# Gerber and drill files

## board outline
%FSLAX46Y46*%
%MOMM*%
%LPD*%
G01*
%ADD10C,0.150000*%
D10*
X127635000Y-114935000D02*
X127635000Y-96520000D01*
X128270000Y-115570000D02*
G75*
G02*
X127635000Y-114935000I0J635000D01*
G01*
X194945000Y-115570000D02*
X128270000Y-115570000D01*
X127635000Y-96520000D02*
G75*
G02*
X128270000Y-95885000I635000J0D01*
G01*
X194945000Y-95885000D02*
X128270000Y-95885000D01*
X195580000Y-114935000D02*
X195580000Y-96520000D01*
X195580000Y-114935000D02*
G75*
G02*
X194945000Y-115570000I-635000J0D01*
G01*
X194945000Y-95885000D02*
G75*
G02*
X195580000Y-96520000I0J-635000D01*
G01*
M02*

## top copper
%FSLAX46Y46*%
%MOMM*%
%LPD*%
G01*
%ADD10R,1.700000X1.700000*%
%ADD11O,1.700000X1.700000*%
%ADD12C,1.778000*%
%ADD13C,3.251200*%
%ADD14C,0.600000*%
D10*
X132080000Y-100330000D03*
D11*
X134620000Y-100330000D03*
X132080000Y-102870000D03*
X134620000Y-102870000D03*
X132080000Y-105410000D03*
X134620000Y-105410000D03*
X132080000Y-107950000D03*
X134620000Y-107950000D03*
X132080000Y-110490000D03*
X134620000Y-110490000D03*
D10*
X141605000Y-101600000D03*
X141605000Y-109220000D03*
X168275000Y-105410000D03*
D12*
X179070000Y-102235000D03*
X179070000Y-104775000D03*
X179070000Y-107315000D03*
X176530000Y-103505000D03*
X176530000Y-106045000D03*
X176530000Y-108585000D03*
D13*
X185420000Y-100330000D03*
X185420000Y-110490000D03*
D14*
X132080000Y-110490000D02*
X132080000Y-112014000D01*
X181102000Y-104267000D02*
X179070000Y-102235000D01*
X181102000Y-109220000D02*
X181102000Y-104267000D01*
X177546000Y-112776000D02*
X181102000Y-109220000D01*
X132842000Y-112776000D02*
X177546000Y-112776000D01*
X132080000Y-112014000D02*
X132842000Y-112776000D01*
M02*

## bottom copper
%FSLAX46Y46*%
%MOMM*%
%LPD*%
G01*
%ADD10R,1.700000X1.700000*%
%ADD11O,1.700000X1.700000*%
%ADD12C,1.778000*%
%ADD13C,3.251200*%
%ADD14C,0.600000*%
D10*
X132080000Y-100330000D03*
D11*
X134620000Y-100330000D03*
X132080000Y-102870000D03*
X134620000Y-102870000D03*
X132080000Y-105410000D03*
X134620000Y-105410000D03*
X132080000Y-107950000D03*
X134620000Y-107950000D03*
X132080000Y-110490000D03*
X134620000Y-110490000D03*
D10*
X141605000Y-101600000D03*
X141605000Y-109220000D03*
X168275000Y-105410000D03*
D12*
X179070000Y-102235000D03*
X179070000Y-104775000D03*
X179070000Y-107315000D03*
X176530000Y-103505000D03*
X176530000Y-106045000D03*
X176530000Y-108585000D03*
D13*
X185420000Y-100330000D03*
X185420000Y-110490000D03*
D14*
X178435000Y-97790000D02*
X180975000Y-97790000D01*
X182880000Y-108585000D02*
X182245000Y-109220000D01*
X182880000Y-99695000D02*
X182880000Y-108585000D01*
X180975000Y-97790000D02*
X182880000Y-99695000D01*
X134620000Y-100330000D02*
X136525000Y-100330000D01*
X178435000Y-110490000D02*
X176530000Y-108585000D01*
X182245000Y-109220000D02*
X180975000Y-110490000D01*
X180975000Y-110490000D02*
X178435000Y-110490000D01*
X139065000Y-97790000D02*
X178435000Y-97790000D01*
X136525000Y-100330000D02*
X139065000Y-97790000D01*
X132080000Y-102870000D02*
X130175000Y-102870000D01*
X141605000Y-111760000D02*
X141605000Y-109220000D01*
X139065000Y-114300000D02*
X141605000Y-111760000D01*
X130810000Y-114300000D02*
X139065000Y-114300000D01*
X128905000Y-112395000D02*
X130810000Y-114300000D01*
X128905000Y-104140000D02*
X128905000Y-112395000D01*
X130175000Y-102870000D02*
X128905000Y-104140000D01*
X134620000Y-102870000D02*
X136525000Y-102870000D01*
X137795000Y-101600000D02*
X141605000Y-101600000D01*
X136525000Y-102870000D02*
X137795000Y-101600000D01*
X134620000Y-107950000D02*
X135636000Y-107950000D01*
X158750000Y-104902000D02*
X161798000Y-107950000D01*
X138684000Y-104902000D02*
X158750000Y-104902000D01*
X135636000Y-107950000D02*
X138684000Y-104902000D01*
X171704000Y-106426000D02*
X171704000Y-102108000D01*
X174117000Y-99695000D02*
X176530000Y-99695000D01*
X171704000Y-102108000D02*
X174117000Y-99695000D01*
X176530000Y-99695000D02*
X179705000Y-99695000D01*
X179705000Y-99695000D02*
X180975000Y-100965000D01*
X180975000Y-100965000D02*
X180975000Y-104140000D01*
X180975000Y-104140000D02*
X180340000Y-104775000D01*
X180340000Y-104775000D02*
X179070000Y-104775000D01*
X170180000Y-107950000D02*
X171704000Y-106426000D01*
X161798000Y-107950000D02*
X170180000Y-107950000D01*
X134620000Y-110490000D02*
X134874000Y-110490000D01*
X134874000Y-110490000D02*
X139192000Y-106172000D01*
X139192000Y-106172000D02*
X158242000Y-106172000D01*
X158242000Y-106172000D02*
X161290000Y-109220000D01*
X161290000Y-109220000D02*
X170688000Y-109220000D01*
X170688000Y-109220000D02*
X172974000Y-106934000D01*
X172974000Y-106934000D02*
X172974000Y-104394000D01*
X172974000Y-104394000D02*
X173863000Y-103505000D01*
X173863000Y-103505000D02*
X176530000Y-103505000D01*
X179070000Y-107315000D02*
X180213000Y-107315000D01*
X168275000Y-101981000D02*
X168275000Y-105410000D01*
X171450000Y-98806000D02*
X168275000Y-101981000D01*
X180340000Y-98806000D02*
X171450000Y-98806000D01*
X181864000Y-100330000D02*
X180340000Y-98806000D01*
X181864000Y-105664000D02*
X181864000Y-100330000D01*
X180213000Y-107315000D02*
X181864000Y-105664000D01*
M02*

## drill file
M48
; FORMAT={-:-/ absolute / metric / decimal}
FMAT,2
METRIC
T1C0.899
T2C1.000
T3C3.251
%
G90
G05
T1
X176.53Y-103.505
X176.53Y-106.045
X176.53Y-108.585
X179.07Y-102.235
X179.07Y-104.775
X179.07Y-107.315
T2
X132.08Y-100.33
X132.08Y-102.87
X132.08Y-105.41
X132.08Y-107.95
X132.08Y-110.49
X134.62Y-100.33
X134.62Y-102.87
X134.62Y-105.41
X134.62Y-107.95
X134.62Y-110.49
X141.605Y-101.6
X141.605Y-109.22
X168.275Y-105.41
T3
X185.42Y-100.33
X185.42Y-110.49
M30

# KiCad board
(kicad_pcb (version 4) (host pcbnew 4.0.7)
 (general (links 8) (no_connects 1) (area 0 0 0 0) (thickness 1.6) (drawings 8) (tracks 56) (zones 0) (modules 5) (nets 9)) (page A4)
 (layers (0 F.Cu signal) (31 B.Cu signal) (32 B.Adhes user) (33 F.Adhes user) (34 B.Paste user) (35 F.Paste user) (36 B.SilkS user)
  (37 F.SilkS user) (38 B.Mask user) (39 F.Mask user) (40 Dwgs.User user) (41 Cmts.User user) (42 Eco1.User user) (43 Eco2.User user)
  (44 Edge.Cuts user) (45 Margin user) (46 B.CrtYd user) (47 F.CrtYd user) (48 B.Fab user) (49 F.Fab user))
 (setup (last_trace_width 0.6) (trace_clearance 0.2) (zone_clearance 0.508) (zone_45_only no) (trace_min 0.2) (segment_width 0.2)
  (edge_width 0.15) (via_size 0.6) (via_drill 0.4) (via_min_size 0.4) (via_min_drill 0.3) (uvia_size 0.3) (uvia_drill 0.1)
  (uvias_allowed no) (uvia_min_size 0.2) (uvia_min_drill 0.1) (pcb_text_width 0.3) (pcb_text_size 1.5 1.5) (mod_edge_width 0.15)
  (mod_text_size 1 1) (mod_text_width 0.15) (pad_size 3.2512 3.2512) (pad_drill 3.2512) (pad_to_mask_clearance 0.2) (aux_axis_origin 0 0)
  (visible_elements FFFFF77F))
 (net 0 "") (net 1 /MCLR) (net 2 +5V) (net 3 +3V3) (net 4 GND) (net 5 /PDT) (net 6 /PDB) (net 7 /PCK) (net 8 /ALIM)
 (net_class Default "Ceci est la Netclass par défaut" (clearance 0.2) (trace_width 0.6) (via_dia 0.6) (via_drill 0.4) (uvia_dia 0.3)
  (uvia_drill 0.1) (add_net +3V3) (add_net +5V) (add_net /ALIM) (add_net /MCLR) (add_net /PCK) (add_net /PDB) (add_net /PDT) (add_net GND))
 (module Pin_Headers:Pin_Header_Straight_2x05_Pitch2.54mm (layer F.Cu) (at 132.08 100.33)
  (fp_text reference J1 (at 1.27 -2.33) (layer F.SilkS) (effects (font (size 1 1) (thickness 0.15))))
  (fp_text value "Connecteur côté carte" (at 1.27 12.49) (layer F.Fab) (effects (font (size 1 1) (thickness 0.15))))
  (pad 1 thru_hole rect (at 0 0) (size 1.7 1.7) (drill 1) (layers *.Cu *.Mask))
  (pad 2 thru_hole oval (at 2.54 0) (size 1.7 1.7) (drill 1) (layers *.Cu *.Mask) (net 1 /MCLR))
  (pad 3 thru_hole oval (at 0 2.54) (size 1.7 1.7) (drill 1) (layers *.Cu *.Mask) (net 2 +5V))
  (pad 4 thru_hole oval (at 2.54 2.54) (size 1.7 1.7) (drill 1) (layers *.Cu *.Mask) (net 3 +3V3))
  (pad 5 thru_hole oval (at 0 5.08) (size 1.7 1.7) (drill 1) (layers *.Cu *.Mask))
  (pad 6 thru_hole oval (at 2.54 5.08) (size 1.7 1.7) (drill 1) (layers *.Cu *.Mask) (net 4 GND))
  (pad 7 thru_hole oval (at 0 7.62) (size 1.7 1.7) (drill 1) (layers *.Cu *.Mask))
  (pad 8 thru_hole oval (at 2.54 7.62) (size 1.7 1.7) (drill 1) (layers *.Cu *.Mask) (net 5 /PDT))
  (pad 9 thru_hole oval (at 0 10.16) (size 1.7 1.7) (drill 1) (layers *.Cu *.Mask) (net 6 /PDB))
  (pad 10 thru_hole oval (at 2.54 10.16) (size 1.7 1.7) (drill 1) (layers *.Cu *.Mask) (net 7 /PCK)))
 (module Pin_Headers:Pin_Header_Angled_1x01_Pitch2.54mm (layer F.Cu) (at 141.605 101.6)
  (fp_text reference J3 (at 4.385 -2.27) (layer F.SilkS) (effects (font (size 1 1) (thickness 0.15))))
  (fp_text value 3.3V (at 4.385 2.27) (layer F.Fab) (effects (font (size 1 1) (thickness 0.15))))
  (pad 1 thru_hole rect (at 0 0) (size 1.7 1.7) (drill 1) (layers *.Cu *.Mask) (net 3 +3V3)))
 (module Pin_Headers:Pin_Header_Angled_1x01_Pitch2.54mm (layer F.Cu) (at 141.605 109.22)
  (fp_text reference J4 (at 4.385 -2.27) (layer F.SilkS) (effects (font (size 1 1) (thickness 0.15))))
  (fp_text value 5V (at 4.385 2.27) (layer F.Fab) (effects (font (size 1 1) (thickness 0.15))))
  (pad 1 thru_hole rect (at 0 0) (size 1.7 1.7) (drill 1) (layers *.Cu *.Mask) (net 2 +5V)))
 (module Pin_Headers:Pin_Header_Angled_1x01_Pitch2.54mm (layer F.Cu) (at 168.275 105.41 180)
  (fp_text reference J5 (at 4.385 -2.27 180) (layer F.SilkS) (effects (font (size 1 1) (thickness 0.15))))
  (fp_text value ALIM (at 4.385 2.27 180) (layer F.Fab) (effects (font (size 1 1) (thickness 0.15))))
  (pad 1 thru_hole rect (at 0 0 180) (size 1.7 1.7) (drill 1) (layers *.Cu *.Mask) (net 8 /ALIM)))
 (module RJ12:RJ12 (layer F.Cu) (at 185.42 105.41 270)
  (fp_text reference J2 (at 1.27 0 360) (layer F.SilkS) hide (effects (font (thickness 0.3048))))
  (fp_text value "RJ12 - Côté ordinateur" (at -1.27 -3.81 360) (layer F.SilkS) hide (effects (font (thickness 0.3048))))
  (pad 6 thru_hole circle (at -3.175 6.35 270) (size 1.778 1.778) (drill 0.89916) (layers *.Cu *.Mask F.SilkS) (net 6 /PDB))
  (pad 4 thru_hole circle (at -0.635 6.35 270) (size 1.778 1.778) (drill 0.89916) (layers *.Cu *.Mask F.SilkS) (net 5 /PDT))
  (pad 2 thru_hole circle (at 1.905 6.35 270) (size 1.778 1.778) (drill 0.89916) (layers *.Cu *.Mask F.SilkS) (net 8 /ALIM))
  (pad 5 thru_hole circle (at -1.905 8.89 270) (size 1.778 1.778) (drill 0.89916) (layers *.Cu *.Mask F.SilkS) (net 7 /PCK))
  (pad 3 thru_hole circle (at 0.635 8.89 270) (size 1.778 1.778) (drill 0.89916) (layers *.Cu *.Mask F.SilkS) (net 4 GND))
  (pad 1 thru_hole circle (at 3.175 8.89 270) (size 1.778 1.778) (drill 0.89916) (layers *.Cu *.Mask F.SilkS) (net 1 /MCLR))
  (pad 8 thru_hole circle (at -5.08 0 270) (size 3.2512 3.2512) (drill 3.2512) (layers *.Cu *.Mask F.SilkS))
  (pad 7 thru_hole circle (at 5.08 0 270) (size 3.2512 3.2512) (drill 3.2512) (layers *.Cu *.Mask F.SilkS)))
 (gr_line (start 127.635 114.935) (end 127.635 96.52) (angle 90) (layer Edge.Cuts) (width 0.15))
 (gr_arc (start 128.27 114.935) (end 128.27 115.57) (angle 90) (layer Edge.Cuts) (width 0.15))
 (gr_line (start 194.945 115.57) (end 128.27 115.57) (angle 90) (layer Edge.Cuts) (width 0.15))
 (gr_arc (start 128.27 96.52) (end 127.635 96.52) (angle 90) (layer Edge.Cuts) (width 0.15))
 (gr_line (start 194.945 95.885) (end 128.27 95.885) (angle 90) (layer Edge.Cuts) (width 0.15))
 (gr_line (start 195.58 114.935) (end 195.58 96.52) (angle 90) (layer Edge.Cuts) (width 0.15))
 (gr_arc (start 194.945 114.935) (end 195.58 114.935) (angle 90) (layer Edge.Cuts) (width 0.15))
 (gr_arc (start 194.945 96.52) (end 194.945 95.885) (angle 90) (layer Edge.Cuts) (width 0.15))
 (segment (start 178.435 97.79) (end 180.975 97.79) (width 0.6) (layer B.Cu) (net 1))
 (segment (start 182.88 108.585) (end 182.245 109.22) (width 0.6) (layer B.Cu) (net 1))
 (segment (start 182.88 99.695) (end 182.88 108.585) (width 0.6) (layer B.Cu) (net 1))
 (segment (start 180.975 97.79) (end 182.88 99.695) (width 0.6) (layer B.Cu) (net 1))
 (segment (start 134.62 100.33) (end 136.525 100.33) (width 0.6) (layer B.Cu) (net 1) (status 400000))
 (segment (start 178.435 110.49) (end 176.53 108.585) (width 0.6) (layer B.Cu) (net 1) (status 800000))
 (segment (start 182.245 109.22) (end 180.975 110.49) (width 0.6) (layer B.Cu) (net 1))
 (segment (start 180.975 110.49) (end 178.435 110.49) (width 0.6) (layer B.Cu) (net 1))
 (segment (start 139.065 97.79) (end 178.435 97.79) (width 0.6) (layer B.Cu) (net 1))
 (segment (start 136.525 100.33) (end 139.065 97.79) (width 0.6) (layer B.Cu) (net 1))
 (segment (start 132.08 102.87) (end 130.175 102.87) (width 0.6) (layer B.Cu) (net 2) (status 400000))
 (segment (start 141.605 111.76) (end 141.605 109.22) (width 0.6) (layer B.Cu) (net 2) (status 800000))
 (segment (start 139.065 114.3) (end 141.605 111.76) (width 0.6) (layer B.Cu) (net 2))
 (segment (start 130.81 114.3) (end 139.065 114.3) (width 0.6) (layer B.Cu) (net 2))
 (segment (start 128.905 112.395) (end 130.81 114.3) (width 0.6) (layer B.Cu) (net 2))
 (segment (start 128.905 104.14) (end 128.905 112.395) (width 0.6) (layer B.Cu) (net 2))
 (segment (start 130.175 102.87) (end 128.905 104.14) (width 0.6) (layer B.Cu) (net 2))
 (segment (start 134.62 102.87) (end 136.525 102.87) (width 0.6) (layer B.Cu) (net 3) (status 400000))
 (segment (start 137.795 101.6) (end 141.605 101.6) (width 0.6) (layer B.Cu) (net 3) (status 800000))
 (segment (start 136.525 102.87) (end 137.795 101.6) (width 0.6) (layer B.Cu) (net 3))
 (segment (start 134.62 107.95) (end 135.636 107.95) (width 0.6) (layer B.Cu) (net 5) (status 400000))
 (segment (start 158.75 104.902) (end 161.798 107.95) (width 0.6) (layer B.Cu) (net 5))
 (segment (start 138.684 104.902) (end 158.75 104.902) (width 0.6) (layer B.Cu) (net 5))
 (segment (start 135.636 107.95) (end 138.684 104.902) (width 0.6) (layer B.Cu) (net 5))
 (segment (start 171.704 106.426) (end 171.704 102.108) (width 0.6) (layer B.Cu) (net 5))
 (segment (start 174.117 99.695) (end 176.53 99.695) (width 0.6) (layer B.Cu) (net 5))
 (segment (start 171.704 102.108) (end 174.117 99.695) (width 0.6) (layer B.Cu) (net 5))
 (segment (start 176.53 99.695) (end 179.705 99.695) (width 0.6) (layer B.Cu) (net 5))
 (segment (start 179.705 99.695) (end 180.975 100.965) (width 0.6) (layer B.Cu) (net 5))
 (segment (start 180.975 100.965) (end 180.975 104.14) (width 0.6) (layer B.Cu) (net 5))
 (segment (start 180.975 104.14) (end 180.34 104.775) (width 0.6) (layer B.Cu) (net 5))
 (segment (start 180.34 104.775) (end 179.07 104.775) (width 0.6) (layer B.Cu) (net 5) (status 800000))
 (segment (start 170.18 107.95) (end 171.704 106.426) (width 0.6) (layer B.Cu) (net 5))
 (segment (start 161.798 107.95) (end 170.18 107.95) (width 0.6) (layer B.Cu) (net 5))
 (segment (start 132.08 110.49) (end 132.08 112.014) (width 0.6) (layer F.Cu) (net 6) (status 400000))
 (segment (start 181.102 104.267) (end 179.07 102.235) (width 0.6) (layer F.Cu) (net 6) (status 800000))
 (segment (start 181.102 109.22) (end 181.102 104.267) (width 0.6) (layer F.Cu) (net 6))
 (segment (start 177.546 112.776) (end 181.102 109.22) (width 0.6) (layer F.Cu) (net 6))
 (segment (start 132.842 112.776) (end 177.546 112.776) (width 0.6) (layer F.Cu) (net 6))
 (segment (start 132.08 112.014) (end 132.842 112.776) (width 0.6) (layer F.Cu) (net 6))
 (segment (start 134.62 110.49) (end 134.874 110.49) (width 0.6) (layer B.Cu) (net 7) (status C00000))
 (segment (start 134.874 110.49) (end 139.192 106.172) (width 0.6) (layer B.Cu) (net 7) (status 400000))
 (segment (start 139.192 106.172) (end 158.242 106.172) (width 0.6) (layer B.Cu) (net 7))
 (segment (start 158.242 106.172) (end 161.29 109.22) (width 0.6) (layer B.Cu) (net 7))
 (segment (start 161.29 109.22) (end 170.688 109.22) (width 0.6) (layer B.Cu) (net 7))
 (segment (start 170.688 109.22) (end 172.974 106.934) (width 0.6) (layer B.Cu) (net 7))
 (segment (start 172.974 106.934) (end 172.974 104.394) (width 0.6) (layer B.Cu) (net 7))
 (segment (start 172.974 104.394) (end 173.863 103.505) (width 0.6) (layer B.Cu) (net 7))
 (segment (start 173.863 103.505) (end 176.53 103.505) (width 0.6) (layer B.Cu) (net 7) (status 800000))
 (segment (start 179.07 107.315) (end 180.213 107.315) (width 0.6) (layer B.Cu) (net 8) (status 400000))
 (segment (start 168.275 101.981) (end 168.275 105.41) (width 0.6) (layer B.Cu) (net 8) (status 800000))
 (segment (start 171.45 98.806) (end 168.275 101.981) (width 0.6) (layer B.Cu) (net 8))
 (segment (start 180.34 98.806) (end 171.45 98.806) (width 0.6) (layer B.Cu) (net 8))
 (segment (start 181.864 100.33) (end 180.34 98.806) (width 0.6) (layer B.Cu) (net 8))
 (segment (start 181.864 105.664) (end 181.864 100.33) (width 0.6) (layer B.Cu) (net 8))
 (segment (start 180.213 107.315) (end 181.864 105.664) (width 0.6) (layer B.Cu) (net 8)))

